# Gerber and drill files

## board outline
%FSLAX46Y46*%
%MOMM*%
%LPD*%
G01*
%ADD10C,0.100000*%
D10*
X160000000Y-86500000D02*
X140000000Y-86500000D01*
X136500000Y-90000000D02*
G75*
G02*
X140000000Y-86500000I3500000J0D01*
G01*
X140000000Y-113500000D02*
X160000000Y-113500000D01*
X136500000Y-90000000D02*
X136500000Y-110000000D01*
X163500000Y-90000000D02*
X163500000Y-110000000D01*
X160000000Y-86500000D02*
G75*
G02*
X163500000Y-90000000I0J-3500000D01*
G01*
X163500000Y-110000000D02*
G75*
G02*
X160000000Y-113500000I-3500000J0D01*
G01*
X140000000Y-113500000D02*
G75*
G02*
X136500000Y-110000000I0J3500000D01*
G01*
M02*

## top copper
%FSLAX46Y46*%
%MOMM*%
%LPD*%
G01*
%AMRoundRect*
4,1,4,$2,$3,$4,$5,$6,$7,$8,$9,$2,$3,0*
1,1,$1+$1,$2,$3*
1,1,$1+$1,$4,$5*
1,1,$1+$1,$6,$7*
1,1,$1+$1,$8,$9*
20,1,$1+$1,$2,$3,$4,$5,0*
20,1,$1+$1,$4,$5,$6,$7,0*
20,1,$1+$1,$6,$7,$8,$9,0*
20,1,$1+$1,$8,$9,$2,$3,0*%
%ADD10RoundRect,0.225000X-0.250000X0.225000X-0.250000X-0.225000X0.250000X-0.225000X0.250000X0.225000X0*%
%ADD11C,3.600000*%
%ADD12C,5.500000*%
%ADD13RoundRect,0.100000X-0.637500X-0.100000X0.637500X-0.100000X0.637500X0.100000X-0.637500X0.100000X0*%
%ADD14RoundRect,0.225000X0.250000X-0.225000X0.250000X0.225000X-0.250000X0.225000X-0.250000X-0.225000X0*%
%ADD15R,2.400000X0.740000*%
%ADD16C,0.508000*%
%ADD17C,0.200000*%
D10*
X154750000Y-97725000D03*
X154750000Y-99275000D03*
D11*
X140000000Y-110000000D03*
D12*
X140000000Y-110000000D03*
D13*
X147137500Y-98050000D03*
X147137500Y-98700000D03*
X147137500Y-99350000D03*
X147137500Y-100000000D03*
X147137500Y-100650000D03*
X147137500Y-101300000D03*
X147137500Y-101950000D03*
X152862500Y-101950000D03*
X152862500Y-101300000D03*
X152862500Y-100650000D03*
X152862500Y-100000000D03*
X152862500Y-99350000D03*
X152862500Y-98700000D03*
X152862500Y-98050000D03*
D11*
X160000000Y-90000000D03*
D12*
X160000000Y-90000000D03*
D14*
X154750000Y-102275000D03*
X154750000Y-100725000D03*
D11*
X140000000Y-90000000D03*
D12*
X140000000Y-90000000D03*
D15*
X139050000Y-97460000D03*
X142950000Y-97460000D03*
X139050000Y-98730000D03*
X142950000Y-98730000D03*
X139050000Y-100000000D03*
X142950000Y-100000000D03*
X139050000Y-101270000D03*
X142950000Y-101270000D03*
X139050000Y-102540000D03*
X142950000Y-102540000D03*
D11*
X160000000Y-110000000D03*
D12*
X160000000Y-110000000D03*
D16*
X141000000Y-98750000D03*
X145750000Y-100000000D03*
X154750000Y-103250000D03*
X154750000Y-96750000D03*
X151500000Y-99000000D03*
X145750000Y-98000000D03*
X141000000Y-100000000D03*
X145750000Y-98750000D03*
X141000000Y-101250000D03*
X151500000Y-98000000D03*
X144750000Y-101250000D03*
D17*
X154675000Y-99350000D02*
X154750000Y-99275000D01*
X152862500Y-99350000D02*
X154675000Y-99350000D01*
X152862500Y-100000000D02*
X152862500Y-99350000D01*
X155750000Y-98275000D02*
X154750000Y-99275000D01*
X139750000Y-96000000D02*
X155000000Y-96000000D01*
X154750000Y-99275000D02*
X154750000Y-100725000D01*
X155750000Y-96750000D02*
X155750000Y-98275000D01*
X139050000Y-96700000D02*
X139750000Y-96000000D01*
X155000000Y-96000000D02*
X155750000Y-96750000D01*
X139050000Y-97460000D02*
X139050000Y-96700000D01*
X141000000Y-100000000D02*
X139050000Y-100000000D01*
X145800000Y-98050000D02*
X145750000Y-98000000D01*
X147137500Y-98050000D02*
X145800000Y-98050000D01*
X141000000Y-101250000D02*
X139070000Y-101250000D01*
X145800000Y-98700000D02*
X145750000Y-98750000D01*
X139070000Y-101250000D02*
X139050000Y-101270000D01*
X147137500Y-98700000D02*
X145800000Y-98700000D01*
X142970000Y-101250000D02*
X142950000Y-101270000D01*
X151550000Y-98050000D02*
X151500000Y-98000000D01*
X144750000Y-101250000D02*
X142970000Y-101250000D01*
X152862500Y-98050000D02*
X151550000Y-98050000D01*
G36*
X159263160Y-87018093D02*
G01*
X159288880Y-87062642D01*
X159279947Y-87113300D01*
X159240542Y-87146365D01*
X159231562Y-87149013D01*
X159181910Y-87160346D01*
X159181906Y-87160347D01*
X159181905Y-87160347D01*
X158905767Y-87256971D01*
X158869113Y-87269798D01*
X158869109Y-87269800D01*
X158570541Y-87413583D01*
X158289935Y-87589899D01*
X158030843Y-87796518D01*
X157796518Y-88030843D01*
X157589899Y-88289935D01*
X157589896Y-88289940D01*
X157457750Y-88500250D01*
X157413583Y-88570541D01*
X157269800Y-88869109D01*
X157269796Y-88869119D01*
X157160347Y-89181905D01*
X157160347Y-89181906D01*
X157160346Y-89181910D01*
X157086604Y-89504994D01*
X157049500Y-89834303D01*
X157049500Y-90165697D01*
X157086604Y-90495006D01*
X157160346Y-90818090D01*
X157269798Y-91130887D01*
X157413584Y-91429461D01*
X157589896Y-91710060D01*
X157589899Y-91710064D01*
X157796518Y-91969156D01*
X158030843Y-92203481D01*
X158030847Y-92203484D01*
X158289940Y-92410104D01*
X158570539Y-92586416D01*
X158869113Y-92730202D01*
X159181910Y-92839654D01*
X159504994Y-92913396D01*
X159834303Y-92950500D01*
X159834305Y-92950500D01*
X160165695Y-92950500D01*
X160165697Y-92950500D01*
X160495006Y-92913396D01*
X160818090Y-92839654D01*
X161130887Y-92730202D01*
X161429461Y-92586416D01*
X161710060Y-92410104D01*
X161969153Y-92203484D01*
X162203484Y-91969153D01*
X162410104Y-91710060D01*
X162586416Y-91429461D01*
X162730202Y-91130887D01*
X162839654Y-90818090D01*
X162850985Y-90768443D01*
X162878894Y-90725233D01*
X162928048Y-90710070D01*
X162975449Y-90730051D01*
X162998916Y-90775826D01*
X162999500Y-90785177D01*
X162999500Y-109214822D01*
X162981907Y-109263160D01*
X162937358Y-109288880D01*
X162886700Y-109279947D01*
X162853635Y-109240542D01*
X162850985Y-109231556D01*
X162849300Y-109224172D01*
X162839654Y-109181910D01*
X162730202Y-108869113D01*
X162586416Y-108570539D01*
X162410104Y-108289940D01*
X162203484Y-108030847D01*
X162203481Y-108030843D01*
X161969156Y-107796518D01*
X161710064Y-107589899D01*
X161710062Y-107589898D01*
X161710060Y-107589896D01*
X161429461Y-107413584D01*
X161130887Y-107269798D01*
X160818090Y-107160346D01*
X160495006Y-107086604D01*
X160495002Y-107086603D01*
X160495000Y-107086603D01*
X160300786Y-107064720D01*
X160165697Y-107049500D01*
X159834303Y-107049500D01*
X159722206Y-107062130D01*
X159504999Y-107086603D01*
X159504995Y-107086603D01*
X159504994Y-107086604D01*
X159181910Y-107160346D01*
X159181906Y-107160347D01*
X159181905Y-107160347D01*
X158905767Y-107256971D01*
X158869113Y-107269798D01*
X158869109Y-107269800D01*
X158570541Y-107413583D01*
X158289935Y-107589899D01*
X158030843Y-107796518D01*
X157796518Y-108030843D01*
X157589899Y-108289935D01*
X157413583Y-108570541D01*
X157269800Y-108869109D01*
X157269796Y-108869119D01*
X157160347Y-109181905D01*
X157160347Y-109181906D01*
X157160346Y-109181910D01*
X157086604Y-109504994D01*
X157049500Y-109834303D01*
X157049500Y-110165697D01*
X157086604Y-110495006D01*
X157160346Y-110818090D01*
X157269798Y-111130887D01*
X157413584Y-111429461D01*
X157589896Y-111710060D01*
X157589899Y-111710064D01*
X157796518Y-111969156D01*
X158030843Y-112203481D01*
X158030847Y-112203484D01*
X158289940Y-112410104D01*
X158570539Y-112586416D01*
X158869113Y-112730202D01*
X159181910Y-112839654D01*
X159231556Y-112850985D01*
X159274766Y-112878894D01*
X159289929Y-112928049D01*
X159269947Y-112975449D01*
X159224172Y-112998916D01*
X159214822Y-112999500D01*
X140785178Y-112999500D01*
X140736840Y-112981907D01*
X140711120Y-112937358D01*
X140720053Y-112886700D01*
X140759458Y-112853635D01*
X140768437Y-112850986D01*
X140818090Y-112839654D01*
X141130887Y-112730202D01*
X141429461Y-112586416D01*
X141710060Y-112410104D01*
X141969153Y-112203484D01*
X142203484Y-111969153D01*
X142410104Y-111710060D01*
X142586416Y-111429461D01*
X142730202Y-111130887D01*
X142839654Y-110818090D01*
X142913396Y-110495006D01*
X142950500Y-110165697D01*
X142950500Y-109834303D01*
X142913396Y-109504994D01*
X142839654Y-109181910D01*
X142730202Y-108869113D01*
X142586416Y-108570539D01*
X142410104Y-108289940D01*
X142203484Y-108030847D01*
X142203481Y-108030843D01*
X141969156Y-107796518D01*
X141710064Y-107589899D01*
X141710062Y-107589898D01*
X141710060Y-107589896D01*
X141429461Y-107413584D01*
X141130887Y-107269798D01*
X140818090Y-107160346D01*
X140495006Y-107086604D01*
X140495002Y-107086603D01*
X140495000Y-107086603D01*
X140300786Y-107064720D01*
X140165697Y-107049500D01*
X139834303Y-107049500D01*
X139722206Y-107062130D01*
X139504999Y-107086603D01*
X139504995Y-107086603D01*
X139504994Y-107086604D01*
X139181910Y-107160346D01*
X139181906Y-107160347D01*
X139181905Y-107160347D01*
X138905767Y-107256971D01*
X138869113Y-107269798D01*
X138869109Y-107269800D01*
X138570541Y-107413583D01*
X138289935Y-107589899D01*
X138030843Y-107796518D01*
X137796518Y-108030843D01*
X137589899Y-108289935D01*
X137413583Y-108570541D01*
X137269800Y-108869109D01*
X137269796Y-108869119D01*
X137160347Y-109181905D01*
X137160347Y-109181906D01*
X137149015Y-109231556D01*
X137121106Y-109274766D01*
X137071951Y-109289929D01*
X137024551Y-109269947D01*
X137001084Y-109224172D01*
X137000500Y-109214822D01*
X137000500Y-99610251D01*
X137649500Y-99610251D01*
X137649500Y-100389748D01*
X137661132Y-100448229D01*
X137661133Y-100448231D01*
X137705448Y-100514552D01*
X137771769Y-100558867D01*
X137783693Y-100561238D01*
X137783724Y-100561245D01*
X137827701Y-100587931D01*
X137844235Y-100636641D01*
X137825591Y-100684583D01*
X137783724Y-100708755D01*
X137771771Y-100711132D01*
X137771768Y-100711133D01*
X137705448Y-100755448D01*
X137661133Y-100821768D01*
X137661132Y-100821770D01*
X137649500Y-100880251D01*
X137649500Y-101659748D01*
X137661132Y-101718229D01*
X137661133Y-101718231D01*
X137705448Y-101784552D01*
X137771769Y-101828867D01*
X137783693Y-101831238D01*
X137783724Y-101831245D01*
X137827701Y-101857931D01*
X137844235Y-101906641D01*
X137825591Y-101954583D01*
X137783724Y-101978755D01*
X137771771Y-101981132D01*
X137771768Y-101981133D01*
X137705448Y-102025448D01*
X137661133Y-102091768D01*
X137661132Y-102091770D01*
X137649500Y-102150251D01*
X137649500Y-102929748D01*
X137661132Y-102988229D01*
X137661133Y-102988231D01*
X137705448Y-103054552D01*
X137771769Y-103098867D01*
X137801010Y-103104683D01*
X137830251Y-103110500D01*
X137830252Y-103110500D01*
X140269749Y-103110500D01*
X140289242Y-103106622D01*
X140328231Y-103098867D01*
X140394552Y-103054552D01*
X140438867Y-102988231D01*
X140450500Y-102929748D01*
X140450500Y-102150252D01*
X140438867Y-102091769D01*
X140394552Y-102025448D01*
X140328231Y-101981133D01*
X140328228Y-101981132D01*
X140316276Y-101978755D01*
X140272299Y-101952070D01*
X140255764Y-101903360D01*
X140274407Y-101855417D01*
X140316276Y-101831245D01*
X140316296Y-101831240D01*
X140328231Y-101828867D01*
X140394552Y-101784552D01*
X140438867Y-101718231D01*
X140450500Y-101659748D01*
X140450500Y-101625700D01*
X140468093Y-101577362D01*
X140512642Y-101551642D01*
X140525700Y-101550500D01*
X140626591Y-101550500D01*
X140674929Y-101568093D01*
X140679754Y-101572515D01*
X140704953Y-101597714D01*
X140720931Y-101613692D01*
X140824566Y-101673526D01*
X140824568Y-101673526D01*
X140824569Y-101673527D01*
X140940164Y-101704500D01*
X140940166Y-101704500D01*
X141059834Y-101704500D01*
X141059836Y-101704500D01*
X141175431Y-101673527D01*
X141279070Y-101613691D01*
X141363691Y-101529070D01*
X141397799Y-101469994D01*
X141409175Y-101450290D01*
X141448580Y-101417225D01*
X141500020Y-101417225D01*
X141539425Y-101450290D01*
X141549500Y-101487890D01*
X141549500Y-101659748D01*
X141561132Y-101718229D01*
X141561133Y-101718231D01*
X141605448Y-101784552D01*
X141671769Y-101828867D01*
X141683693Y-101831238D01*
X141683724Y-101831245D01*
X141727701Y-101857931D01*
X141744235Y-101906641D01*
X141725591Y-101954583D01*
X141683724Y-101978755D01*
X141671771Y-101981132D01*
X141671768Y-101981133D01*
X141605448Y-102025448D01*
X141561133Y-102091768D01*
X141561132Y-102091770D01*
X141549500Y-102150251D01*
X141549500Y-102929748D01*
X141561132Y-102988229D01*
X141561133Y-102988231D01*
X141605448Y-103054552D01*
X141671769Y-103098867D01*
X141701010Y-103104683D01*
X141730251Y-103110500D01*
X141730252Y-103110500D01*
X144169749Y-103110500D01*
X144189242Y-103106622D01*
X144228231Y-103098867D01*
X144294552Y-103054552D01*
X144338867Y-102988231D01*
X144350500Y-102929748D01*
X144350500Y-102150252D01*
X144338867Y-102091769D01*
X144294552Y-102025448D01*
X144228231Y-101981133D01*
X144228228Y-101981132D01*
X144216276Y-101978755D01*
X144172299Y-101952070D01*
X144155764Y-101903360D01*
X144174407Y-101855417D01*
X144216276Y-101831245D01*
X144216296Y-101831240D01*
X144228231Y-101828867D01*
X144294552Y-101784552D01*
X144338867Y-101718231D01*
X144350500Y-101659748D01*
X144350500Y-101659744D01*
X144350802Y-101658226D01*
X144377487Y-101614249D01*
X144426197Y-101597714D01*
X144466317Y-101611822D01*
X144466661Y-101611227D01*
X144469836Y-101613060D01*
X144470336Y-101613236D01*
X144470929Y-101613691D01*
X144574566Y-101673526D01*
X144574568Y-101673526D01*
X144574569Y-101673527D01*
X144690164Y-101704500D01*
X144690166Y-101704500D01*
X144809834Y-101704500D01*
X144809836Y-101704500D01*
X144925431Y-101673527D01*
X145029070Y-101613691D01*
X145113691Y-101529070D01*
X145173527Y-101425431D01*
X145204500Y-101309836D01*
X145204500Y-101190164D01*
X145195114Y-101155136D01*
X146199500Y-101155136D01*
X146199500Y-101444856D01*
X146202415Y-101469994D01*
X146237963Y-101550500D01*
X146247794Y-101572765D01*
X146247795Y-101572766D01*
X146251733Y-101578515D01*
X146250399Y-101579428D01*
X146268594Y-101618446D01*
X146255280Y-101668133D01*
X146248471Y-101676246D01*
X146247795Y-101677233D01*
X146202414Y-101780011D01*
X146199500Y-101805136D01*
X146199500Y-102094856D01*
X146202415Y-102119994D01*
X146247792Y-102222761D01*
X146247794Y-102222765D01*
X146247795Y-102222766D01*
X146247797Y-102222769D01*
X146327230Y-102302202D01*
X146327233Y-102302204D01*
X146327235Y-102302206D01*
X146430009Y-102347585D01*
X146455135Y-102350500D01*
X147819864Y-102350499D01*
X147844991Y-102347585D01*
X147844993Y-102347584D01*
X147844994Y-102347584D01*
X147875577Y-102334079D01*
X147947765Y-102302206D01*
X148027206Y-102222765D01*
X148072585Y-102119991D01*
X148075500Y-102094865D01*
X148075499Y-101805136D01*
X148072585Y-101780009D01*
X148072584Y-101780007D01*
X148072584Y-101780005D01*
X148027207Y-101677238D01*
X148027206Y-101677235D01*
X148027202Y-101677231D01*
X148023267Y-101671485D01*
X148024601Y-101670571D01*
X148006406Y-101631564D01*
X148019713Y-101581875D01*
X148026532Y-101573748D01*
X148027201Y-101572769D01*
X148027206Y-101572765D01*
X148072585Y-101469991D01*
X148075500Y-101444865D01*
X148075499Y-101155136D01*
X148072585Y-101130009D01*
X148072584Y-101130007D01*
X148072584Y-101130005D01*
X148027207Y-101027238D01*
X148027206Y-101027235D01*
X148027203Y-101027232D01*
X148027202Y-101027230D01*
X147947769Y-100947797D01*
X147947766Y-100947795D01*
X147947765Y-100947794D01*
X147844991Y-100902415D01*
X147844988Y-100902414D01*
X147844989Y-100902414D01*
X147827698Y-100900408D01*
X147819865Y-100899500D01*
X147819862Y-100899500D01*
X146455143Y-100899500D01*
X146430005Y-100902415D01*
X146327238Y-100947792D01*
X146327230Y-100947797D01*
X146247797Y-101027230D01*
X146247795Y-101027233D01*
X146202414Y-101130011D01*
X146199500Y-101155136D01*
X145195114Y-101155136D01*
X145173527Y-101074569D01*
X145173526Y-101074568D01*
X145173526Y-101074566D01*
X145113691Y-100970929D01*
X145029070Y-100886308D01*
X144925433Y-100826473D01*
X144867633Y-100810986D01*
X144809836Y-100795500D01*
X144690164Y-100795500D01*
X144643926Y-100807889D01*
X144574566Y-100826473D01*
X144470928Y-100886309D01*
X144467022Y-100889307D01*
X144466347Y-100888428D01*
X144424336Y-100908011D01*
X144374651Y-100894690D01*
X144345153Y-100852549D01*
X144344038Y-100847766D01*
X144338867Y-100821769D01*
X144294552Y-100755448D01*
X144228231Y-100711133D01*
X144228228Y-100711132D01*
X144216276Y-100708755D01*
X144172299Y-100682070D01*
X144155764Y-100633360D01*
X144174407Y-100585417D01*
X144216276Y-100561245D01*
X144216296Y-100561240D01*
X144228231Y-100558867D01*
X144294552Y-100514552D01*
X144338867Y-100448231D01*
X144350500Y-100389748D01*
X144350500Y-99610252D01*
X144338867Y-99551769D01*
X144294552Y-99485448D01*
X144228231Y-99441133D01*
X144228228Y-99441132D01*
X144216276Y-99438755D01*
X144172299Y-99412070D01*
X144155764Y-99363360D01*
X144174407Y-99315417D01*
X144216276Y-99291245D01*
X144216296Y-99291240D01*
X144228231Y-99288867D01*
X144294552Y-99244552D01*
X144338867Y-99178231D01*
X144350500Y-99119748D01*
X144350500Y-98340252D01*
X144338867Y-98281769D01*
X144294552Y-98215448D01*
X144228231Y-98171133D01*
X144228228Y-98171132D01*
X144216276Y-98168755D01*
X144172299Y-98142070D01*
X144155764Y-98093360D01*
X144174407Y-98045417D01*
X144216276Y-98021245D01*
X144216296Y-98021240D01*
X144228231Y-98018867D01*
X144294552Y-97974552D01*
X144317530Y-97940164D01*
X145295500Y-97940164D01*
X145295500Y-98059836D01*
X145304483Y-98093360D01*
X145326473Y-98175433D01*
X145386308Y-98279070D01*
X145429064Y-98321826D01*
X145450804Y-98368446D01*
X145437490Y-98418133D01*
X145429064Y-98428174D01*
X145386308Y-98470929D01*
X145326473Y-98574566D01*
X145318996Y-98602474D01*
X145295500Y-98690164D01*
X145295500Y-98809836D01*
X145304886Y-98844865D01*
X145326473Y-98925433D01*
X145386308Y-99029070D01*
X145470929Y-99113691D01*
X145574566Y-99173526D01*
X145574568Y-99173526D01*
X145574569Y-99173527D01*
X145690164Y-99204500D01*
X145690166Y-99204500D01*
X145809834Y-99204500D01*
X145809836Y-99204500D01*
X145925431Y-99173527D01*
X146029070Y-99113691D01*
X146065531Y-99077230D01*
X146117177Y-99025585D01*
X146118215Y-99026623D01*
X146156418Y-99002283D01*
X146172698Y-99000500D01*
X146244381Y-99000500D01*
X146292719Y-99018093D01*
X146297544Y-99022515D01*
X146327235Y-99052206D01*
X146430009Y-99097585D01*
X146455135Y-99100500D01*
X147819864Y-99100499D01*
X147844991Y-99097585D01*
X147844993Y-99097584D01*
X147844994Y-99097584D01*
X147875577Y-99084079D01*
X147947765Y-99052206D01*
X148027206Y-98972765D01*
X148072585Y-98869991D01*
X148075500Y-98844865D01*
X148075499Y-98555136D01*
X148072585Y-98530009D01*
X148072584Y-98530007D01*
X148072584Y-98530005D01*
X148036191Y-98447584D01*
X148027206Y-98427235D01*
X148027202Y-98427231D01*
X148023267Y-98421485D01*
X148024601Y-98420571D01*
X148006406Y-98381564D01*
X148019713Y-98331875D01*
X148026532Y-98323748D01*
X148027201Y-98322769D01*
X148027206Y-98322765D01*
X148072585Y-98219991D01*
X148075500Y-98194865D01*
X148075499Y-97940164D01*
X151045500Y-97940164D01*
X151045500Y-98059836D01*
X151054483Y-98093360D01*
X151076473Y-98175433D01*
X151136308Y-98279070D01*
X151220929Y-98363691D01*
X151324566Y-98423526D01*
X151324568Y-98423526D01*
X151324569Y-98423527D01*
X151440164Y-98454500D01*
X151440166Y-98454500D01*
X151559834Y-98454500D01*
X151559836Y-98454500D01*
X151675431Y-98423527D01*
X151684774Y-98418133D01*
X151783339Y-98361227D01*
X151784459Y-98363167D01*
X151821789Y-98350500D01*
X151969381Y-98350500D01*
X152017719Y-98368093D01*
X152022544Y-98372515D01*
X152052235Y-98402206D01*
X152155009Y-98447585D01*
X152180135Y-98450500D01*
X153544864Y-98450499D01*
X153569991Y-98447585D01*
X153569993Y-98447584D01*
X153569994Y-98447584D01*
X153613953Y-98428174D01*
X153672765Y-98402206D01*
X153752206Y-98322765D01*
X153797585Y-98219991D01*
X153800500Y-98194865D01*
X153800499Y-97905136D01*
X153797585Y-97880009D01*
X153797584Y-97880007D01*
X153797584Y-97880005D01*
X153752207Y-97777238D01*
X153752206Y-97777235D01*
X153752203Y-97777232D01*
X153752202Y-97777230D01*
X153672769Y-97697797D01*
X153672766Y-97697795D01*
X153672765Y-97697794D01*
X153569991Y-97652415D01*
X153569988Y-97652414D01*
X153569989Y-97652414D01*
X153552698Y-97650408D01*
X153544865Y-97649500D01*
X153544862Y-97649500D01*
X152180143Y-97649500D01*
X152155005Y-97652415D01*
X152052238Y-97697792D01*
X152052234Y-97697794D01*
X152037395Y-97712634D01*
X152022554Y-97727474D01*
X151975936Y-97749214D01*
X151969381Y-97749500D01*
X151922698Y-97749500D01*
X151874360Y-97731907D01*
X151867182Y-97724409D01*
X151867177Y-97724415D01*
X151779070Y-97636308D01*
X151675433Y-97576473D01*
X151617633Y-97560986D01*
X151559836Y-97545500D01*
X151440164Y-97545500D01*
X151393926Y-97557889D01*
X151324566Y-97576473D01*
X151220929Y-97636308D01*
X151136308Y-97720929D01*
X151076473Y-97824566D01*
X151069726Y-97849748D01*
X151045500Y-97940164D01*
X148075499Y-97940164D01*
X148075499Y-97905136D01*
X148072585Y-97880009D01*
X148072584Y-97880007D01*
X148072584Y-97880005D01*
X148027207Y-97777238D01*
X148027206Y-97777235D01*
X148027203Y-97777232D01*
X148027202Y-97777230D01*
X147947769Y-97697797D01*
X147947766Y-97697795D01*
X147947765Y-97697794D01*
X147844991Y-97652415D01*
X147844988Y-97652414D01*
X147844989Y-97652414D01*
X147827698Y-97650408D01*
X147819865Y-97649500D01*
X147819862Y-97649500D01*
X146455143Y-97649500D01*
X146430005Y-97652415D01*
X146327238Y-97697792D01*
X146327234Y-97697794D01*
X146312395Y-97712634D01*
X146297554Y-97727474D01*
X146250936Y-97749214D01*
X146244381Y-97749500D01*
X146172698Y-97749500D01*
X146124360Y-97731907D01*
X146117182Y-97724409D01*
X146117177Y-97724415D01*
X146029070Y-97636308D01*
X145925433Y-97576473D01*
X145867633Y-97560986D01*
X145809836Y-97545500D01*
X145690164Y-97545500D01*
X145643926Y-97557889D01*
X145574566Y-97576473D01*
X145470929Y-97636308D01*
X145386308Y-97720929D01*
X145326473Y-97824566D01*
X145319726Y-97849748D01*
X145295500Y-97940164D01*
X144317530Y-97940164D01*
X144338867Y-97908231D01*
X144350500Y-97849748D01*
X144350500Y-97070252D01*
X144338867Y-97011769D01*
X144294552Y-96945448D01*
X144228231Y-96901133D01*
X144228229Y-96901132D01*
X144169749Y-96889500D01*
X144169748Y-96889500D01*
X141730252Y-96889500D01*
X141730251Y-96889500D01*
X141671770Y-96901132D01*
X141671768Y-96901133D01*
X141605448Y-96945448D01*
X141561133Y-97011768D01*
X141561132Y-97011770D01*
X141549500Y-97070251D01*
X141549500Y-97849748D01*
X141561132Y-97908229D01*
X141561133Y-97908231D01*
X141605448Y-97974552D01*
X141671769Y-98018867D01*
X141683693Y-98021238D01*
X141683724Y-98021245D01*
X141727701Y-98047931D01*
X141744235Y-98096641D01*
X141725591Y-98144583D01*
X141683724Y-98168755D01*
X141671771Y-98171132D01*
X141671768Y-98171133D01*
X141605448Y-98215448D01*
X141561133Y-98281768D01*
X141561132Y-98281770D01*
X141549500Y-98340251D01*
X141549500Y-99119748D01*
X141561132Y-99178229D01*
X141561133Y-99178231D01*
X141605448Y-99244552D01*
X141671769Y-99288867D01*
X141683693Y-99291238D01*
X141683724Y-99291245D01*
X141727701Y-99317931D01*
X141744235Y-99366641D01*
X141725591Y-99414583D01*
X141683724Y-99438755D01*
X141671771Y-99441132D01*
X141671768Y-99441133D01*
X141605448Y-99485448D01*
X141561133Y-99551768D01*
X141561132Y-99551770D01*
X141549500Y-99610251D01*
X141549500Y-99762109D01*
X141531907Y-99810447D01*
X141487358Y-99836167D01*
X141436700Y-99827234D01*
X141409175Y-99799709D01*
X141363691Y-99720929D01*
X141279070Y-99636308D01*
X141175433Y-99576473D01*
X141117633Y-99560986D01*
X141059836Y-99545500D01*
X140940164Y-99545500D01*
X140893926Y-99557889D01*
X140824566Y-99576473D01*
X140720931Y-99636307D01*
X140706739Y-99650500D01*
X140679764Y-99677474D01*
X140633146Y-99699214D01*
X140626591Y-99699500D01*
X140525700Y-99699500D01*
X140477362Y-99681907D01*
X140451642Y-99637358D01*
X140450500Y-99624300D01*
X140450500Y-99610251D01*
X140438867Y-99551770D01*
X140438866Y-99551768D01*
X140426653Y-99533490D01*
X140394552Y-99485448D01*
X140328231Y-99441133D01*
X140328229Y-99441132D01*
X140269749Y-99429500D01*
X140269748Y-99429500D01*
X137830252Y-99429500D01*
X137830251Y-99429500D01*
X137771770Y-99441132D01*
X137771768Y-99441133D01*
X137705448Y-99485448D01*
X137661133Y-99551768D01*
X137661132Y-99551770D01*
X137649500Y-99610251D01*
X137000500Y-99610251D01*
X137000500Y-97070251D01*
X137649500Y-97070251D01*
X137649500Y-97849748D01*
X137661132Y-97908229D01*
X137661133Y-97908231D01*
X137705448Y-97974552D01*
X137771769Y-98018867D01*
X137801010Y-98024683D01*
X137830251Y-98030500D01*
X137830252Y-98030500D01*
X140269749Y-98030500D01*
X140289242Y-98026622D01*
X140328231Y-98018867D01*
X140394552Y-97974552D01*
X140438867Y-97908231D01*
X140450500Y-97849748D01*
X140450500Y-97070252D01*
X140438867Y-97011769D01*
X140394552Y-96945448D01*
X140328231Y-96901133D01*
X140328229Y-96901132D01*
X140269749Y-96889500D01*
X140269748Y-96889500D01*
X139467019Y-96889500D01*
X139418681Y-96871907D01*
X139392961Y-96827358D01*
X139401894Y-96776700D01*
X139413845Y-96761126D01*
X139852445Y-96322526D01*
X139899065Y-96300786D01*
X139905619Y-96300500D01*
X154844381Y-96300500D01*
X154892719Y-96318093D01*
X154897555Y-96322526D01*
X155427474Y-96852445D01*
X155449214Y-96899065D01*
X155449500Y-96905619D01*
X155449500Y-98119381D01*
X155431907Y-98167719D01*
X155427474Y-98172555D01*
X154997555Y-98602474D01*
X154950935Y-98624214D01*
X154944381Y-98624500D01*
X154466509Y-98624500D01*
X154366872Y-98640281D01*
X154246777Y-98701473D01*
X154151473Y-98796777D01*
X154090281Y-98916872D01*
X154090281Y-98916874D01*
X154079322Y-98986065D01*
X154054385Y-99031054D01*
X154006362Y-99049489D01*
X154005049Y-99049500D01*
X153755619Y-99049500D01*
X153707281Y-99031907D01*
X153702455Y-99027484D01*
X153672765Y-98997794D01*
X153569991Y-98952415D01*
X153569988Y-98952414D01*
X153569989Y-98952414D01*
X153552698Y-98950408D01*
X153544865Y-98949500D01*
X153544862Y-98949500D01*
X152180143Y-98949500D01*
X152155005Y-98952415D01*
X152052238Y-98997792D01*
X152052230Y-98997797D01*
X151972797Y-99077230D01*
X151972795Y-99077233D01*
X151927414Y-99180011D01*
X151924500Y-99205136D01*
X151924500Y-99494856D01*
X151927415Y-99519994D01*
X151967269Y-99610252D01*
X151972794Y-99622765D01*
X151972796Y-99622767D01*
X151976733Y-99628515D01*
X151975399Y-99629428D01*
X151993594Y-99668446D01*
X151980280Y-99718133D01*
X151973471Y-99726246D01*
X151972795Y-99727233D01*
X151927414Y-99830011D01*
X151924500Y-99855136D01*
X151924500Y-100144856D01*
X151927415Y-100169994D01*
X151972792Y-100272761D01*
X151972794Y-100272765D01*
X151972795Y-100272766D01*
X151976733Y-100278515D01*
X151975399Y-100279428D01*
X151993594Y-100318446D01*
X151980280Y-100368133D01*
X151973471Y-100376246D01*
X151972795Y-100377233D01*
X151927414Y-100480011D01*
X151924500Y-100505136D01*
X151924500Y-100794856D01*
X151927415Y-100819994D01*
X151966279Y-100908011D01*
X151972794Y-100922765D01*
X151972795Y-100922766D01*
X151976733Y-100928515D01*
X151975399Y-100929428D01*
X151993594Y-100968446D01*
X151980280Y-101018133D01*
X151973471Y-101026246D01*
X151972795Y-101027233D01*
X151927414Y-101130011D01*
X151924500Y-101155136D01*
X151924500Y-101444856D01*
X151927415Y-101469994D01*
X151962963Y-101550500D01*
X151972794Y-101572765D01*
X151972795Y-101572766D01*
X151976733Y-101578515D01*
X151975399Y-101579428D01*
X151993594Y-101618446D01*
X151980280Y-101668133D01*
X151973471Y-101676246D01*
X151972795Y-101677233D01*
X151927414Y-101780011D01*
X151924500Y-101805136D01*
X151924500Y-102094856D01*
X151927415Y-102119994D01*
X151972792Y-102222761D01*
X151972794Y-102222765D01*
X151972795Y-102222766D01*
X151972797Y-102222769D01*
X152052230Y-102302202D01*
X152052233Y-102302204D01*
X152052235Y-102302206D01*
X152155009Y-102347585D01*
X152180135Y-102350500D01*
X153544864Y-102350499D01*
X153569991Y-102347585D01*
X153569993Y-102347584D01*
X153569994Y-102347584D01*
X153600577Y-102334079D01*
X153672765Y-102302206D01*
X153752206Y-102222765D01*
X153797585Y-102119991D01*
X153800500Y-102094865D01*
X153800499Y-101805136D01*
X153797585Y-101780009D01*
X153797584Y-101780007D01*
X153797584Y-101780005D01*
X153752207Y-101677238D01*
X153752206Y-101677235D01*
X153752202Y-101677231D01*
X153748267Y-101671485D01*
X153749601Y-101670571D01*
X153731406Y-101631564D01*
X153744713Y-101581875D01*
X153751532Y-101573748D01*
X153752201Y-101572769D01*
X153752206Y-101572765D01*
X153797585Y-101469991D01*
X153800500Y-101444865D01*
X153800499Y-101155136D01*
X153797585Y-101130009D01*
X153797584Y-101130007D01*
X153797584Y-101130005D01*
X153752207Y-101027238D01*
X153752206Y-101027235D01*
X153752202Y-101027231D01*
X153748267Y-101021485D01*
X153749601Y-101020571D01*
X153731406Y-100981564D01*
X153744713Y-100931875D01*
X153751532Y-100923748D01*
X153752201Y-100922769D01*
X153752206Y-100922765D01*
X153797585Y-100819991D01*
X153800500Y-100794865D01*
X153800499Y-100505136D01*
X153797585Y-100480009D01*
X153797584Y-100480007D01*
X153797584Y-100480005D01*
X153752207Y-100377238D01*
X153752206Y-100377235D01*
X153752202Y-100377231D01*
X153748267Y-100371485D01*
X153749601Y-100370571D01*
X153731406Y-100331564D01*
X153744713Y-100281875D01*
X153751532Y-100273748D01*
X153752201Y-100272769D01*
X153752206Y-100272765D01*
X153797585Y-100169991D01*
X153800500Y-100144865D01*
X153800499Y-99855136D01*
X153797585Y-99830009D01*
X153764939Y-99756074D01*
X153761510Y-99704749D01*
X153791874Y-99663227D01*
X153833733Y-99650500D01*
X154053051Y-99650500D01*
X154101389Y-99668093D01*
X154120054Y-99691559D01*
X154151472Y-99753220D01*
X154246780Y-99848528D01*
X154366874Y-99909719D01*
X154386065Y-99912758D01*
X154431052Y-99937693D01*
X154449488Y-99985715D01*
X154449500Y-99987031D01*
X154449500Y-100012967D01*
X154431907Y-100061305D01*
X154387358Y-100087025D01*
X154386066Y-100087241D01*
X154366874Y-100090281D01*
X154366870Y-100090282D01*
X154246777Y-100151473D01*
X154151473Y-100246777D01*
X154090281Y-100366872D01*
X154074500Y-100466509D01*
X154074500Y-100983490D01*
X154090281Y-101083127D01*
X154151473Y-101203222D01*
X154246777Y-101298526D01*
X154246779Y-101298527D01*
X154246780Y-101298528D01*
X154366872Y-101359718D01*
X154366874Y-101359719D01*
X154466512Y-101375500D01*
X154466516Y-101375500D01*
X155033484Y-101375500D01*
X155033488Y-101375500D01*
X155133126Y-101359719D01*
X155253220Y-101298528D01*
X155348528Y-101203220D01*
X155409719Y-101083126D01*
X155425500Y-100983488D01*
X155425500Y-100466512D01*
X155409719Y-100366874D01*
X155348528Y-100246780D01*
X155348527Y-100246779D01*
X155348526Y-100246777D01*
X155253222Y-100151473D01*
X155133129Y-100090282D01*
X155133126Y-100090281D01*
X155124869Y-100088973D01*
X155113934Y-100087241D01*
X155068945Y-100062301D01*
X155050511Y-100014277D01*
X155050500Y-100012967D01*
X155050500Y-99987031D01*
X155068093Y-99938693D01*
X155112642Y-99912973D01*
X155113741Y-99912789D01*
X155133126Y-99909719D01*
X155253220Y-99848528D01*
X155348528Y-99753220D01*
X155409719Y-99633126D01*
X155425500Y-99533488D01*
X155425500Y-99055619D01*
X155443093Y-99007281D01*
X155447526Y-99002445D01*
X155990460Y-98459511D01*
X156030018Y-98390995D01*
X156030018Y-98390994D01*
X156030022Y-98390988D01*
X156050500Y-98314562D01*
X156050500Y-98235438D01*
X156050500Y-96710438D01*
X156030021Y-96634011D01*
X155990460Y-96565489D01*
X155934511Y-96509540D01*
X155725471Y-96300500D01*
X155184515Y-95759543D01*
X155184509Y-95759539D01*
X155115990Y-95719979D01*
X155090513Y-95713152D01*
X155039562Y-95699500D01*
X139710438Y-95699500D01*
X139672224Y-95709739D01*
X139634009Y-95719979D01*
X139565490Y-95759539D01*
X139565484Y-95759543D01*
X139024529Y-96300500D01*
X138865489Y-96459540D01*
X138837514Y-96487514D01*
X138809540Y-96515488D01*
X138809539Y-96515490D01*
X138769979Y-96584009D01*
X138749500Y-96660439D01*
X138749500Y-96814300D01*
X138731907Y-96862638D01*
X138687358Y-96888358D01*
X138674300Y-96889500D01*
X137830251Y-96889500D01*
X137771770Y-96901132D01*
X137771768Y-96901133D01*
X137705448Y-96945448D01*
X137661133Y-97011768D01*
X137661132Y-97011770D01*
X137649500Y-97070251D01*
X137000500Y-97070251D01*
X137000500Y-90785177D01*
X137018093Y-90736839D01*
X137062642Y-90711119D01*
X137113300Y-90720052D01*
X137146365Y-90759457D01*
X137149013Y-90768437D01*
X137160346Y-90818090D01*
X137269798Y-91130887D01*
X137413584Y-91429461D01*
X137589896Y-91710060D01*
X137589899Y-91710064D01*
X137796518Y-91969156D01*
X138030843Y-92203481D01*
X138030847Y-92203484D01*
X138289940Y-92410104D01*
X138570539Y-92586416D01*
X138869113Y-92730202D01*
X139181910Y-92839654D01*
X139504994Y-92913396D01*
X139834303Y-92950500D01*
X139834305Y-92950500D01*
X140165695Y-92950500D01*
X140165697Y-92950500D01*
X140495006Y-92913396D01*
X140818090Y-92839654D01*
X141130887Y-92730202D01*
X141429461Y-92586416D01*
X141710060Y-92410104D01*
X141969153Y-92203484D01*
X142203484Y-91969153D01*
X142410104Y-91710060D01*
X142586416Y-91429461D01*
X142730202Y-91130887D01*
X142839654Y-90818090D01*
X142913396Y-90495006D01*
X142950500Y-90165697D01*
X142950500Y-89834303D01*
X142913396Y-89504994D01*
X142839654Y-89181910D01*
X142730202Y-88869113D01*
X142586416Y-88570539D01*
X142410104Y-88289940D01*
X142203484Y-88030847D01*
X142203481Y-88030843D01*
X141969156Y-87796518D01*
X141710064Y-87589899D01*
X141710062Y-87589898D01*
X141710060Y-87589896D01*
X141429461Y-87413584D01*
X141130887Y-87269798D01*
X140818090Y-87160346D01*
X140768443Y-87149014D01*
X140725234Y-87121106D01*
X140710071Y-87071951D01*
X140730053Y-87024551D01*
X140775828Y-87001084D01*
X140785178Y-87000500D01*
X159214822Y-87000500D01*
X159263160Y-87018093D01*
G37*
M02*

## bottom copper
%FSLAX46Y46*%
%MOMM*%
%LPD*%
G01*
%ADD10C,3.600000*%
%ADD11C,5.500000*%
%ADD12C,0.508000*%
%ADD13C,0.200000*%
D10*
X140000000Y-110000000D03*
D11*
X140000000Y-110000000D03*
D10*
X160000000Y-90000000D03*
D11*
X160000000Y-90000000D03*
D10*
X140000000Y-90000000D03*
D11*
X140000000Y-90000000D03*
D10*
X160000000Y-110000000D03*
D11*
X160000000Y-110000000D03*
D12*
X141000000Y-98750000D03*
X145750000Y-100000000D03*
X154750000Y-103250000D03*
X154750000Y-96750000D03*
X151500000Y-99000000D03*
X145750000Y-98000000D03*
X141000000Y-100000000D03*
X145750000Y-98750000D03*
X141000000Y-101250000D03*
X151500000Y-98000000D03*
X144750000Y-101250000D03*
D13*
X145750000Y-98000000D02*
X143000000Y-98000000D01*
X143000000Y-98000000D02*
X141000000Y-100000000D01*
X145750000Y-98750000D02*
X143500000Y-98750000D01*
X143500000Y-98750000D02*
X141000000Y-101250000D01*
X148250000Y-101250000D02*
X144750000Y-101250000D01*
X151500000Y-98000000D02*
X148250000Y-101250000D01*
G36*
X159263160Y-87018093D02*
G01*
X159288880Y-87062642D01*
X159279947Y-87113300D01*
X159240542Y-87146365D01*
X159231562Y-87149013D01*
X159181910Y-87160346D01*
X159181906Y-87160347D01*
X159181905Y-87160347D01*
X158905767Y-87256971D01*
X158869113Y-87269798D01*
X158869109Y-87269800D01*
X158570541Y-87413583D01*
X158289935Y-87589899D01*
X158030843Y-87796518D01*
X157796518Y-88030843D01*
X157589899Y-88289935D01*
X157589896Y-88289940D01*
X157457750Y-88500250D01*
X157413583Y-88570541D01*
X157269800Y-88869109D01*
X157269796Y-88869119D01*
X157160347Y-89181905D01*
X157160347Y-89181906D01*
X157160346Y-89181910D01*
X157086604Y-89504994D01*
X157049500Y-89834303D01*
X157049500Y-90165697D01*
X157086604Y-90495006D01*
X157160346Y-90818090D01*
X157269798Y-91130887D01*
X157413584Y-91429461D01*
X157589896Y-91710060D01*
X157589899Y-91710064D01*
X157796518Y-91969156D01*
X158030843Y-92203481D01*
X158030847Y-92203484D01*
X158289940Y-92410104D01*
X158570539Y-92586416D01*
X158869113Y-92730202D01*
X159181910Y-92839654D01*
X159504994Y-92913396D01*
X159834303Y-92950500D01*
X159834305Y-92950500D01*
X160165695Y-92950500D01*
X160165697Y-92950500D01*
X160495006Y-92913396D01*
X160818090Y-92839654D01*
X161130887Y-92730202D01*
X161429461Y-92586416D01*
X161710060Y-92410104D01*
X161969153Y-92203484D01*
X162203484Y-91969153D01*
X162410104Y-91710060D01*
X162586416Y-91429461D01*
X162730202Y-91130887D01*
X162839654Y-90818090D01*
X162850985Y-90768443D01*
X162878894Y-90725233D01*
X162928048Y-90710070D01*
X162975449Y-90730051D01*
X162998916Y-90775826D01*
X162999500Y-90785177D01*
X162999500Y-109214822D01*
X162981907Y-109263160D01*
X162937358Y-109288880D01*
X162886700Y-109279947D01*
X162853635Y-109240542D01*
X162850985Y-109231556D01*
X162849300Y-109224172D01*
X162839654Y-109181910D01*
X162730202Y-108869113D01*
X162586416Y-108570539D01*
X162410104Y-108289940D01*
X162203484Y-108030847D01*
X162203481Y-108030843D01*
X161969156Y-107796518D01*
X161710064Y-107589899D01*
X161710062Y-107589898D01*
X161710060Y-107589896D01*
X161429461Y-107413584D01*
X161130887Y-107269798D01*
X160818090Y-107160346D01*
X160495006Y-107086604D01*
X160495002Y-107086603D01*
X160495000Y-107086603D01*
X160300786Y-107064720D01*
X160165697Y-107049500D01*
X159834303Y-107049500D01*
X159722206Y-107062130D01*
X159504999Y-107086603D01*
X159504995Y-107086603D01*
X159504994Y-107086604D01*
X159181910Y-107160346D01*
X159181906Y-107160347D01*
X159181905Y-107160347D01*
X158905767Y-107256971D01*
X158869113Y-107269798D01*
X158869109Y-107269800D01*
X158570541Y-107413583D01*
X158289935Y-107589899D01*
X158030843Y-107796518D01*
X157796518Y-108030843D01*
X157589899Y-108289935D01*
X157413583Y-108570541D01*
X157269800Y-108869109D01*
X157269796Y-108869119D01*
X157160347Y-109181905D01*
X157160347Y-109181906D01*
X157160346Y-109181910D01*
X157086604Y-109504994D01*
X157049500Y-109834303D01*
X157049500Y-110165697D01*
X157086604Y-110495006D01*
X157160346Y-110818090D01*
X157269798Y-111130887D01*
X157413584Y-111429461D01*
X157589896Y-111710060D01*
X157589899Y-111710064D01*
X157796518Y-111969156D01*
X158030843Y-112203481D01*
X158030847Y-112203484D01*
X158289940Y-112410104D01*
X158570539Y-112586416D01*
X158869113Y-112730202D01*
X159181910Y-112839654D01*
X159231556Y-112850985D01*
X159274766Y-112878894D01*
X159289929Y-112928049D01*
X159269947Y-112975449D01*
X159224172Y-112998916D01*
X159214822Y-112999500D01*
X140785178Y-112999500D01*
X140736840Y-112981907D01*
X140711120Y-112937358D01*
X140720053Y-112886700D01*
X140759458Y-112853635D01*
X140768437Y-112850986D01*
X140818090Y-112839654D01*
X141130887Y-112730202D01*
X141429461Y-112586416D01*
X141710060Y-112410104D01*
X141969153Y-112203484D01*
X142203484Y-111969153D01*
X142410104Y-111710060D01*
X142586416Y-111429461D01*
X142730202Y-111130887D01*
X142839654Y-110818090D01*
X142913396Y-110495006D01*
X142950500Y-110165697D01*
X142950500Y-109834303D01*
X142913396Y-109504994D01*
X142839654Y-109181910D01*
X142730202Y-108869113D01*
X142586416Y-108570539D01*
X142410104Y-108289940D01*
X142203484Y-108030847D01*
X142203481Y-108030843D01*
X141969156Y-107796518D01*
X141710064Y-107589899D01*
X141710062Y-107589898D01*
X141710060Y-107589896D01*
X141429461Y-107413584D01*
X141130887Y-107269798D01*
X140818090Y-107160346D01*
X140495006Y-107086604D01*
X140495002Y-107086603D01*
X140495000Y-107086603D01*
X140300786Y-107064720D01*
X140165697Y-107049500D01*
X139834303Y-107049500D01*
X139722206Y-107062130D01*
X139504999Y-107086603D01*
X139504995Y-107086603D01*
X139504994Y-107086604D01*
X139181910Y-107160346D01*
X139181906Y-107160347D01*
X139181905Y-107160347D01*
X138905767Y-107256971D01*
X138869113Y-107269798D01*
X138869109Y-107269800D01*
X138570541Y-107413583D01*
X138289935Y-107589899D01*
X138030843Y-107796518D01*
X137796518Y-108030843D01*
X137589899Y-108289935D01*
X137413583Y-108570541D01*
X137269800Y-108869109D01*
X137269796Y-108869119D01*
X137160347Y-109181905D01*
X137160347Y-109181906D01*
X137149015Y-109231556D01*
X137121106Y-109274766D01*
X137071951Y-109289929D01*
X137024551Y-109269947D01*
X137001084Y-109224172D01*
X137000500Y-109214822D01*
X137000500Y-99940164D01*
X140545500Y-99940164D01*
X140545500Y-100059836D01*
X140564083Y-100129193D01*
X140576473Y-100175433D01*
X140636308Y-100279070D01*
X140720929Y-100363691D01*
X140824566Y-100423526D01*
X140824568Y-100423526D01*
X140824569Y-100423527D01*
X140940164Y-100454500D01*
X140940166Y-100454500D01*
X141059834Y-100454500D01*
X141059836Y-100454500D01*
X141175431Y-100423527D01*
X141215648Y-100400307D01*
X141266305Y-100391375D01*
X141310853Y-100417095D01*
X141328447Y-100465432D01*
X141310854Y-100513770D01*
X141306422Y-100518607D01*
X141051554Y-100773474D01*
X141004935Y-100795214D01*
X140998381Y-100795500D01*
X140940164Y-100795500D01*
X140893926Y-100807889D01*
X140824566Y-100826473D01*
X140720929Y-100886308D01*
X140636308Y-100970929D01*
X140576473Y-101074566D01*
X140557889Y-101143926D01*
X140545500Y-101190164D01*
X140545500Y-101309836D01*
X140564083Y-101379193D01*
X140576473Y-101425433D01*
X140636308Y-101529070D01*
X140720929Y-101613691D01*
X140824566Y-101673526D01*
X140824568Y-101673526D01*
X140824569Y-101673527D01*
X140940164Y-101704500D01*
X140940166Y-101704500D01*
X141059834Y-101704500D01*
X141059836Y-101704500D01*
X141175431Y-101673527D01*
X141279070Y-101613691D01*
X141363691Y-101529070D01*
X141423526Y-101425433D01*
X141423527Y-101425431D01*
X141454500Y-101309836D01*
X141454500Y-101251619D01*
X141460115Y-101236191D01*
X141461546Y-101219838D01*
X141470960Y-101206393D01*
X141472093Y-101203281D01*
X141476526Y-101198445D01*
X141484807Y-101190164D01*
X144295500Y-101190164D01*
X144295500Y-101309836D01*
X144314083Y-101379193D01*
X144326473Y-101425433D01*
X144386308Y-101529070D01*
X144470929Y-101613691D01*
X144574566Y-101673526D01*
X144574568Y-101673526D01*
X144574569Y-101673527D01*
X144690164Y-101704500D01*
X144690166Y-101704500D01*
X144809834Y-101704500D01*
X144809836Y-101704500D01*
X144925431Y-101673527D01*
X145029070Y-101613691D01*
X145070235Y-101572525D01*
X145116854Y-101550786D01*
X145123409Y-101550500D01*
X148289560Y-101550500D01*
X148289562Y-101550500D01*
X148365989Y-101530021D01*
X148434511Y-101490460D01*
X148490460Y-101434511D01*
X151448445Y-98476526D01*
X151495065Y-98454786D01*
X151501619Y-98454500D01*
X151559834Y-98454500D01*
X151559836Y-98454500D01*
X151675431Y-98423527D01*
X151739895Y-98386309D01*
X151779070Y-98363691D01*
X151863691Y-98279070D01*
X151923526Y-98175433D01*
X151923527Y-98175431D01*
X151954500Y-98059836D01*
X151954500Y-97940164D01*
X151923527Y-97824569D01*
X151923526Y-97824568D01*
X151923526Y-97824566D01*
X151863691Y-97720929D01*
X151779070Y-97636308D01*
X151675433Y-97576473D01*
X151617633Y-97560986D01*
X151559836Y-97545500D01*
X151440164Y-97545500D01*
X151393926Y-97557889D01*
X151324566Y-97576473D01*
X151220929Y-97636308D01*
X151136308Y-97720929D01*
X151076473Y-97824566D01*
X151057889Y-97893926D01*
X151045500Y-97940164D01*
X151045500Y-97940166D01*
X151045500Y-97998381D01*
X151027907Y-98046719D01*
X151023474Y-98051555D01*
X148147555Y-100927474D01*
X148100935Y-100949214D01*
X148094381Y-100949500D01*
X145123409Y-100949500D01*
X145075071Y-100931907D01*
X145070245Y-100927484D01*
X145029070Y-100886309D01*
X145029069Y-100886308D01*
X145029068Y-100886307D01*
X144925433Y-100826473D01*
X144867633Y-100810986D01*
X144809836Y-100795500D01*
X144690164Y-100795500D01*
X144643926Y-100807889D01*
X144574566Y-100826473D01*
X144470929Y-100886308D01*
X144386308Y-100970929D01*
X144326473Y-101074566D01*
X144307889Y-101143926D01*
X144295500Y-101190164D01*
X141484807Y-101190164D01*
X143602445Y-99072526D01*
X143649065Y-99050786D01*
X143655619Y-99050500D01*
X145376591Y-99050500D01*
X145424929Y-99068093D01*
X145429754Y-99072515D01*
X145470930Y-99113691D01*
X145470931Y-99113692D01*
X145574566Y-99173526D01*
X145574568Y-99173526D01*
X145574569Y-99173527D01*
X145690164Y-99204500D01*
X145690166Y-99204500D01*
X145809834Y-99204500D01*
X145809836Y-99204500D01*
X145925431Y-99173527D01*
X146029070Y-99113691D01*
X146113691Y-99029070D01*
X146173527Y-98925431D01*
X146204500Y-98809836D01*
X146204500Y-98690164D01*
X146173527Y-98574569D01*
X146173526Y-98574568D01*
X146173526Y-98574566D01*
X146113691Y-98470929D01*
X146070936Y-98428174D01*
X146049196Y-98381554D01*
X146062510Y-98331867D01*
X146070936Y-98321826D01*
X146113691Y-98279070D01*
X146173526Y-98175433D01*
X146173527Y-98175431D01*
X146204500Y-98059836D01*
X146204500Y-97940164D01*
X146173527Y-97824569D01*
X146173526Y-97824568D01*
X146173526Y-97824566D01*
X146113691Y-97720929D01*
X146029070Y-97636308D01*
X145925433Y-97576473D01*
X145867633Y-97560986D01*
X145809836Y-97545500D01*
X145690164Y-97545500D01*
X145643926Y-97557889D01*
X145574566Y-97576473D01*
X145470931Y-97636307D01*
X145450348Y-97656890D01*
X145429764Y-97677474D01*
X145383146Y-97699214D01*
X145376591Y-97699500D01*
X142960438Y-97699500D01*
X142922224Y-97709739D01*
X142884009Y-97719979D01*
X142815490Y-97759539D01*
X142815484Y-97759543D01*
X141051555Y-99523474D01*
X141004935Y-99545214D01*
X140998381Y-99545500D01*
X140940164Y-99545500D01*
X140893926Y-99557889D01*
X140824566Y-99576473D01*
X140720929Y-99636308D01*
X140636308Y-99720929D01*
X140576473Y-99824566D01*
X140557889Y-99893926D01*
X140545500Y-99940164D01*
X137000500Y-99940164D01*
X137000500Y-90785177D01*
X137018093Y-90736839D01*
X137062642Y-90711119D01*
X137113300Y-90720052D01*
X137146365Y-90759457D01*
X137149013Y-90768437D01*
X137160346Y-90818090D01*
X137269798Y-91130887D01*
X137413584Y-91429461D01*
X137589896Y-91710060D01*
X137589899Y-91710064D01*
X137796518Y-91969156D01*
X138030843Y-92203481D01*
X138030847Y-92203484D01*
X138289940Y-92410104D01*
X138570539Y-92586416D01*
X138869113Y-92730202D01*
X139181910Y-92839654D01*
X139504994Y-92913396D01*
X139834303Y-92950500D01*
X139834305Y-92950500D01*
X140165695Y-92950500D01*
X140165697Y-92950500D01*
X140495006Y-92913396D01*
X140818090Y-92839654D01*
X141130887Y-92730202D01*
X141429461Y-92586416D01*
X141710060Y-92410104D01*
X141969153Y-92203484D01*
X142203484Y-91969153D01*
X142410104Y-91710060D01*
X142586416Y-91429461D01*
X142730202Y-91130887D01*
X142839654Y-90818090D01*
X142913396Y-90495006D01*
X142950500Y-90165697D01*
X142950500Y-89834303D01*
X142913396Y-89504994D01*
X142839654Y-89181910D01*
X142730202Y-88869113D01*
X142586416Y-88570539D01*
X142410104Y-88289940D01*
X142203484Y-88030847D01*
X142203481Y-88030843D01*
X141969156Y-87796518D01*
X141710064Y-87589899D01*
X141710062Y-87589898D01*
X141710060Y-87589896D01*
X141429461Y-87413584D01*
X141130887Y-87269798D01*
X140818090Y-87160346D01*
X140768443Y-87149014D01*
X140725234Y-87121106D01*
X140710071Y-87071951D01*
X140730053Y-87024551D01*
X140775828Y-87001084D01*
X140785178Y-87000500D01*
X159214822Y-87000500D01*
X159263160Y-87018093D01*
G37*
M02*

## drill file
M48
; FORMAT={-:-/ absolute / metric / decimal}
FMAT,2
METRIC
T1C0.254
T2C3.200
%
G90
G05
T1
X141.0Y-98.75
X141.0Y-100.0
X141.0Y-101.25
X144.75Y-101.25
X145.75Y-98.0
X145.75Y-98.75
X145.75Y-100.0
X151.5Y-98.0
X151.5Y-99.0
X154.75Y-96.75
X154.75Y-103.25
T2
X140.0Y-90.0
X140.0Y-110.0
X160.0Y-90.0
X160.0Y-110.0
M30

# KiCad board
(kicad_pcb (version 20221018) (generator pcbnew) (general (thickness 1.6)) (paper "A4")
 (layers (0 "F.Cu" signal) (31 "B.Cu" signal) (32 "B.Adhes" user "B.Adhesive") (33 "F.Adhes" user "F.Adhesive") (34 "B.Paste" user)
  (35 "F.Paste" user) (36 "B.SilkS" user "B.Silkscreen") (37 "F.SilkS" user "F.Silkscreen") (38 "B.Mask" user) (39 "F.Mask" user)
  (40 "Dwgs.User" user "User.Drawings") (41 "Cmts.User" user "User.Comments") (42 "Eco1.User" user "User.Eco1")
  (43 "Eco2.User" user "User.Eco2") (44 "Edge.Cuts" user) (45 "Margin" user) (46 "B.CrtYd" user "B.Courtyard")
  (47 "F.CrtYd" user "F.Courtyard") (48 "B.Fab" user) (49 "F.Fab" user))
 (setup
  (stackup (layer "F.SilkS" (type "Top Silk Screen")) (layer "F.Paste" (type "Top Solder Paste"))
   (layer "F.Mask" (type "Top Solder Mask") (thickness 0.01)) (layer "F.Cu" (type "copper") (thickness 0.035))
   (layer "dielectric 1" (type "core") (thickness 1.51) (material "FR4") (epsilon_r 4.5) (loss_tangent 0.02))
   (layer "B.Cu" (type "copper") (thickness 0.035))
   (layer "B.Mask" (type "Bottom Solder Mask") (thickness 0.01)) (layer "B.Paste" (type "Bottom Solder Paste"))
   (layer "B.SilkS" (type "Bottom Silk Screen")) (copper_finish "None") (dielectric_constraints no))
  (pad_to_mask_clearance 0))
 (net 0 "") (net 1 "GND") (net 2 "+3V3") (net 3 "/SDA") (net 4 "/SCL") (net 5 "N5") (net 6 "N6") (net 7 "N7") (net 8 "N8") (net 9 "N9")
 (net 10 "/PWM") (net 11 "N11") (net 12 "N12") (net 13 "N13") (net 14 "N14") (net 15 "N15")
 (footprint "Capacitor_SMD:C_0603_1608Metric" (layer "F.Cu") (at 154.75 98.5 -90)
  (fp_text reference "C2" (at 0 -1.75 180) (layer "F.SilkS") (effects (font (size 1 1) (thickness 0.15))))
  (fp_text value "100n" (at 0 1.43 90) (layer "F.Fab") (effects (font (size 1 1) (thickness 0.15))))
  (pad "1" smd roundrect (at -0.775 0 270) (size 0.9 0.95) (layers "F.Cu" "F.Paste" "F.Mask") (roundrect_rratio 0.25) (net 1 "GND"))
  (pad "2" smd roundrect (at 0.775 0 270) (size 0.9 0.95) (layers "F.Cu" "F.Paste" "F.Mask") (roundrect_rratio 0.25) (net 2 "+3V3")))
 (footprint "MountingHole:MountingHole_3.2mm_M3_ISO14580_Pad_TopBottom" (layer "F.Cu") (at 140 110)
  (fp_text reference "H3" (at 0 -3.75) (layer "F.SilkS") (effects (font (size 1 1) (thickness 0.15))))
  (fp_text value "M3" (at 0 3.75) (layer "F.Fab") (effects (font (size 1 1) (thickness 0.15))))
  (pad "1" thru_hole circle (at 0 0) (size 3.6 3.6) (drill 3.2) (layers "*.Cu" "*.Mask"))
  (pad "1" connect circle (at 0 0) (size 5.5 5.5) (layers "F.Cu" "F.Mask"))
  (pad "1" connect circle (at 0 0) (size 5.5 5.5) (layers "B.Cu" "B.Mask")))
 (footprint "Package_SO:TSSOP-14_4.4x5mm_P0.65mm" (layer "F.Cu") (at 150 100)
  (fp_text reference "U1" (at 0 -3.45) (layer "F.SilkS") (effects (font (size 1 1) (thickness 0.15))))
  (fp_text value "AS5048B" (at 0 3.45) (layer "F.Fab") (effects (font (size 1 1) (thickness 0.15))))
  (pad "1" smd roundrect (at -2.8625 -1.95) (size 1.475 0.4) (layers "F.Cu" "F.Paste" "F.Mask") (roundrect_rratio 0.25) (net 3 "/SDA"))
  (pad "2" smd roundrect (at -2.8625 -1.3) (size 1.475 0.4) (layers "F.Cu" "F.Paste" "F.Mask") (roundrect_rratio 0.25) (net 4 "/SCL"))
  (pad "3" smd roundrect (at -2.8625 -0.65) (size 1.475 0.4) (layers "F.Cu" "F.Paste" "F.Mask") (roundrect_rratio 0.25) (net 1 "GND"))
  (pad "4" smd roundrect (at -2.8625 0) (size 1.475 0.4) (layers "F.Cu" "F.Paste" "F.Mask") (roundrect_rratio 0.25) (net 1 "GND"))
  (pad "5" smd roundrect (at -2.8625 0.65) (size 1.475 0.4) (layers "F.Cu" "F.Paste" "F.Mask") (roundrect_rratio 0.25) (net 1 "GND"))
  (pad "6" smd roundrect (at -2.8625 1.3) (size 1.475 0.4) (layers "F.Cu" "F.Paste" "F.Mask") (roundrect_rratio 0.25) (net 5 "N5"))
  (pad "7" smd roundrect (at -2.8625 1.95) (size 1.475 0.4) (layers "F.Cu" "F.Paste" "F.Mask") (roundrect_rratio 0.25) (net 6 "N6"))
  (pad "8" smd roundrect (at 2.8625 1.95) (size 1.475 0.4) (layers "F.Cu" "F.Paste" "F.Mask") (roundrect_rratio 0.25) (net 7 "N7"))
  (pad "9" smd roundrect (at 2.8625 1.3) (size 1.475 0.4) (layers "F.Cu" "F.Paste" "F.Mask") (roundrect_rratio 0.25) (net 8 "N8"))
  (pad "10" smd roundrect (at 2.8625 0.65) (size 1.475 0.4) (layers "F.Cu" "F.Paste" "F.Mask") (roundrect_rratio 0.25) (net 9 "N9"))
  (pad "11" smd roundrect (at 2.8625 0) (size 1.475 0.4) (layers "F.Cu" "F.Paste" "F.Mask") (roundrect_rratio 0.25) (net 2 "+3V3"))
  (pad "12" smd roundrect (at 2.8625 -0.65) (size 1.475 0.4) (layers "F.Cu" "F.Paste" "F.Mask") (roundrect_rratio 0.25) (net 2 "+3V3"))
  (pad "13" smd roundrect (at 2.8625 -1.3) (size 1.475 0.4) (layers "F.Cu" "F.Paste" "F.Mask") (roundrect_rratio 0.25) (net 1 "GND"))
  (pad "14" smd roundrect (at 2.8625 -1.95) (size 1.475 0.4) (layers "F.Cu" "F.Paste" "F.Mask") (roundrect_rratio 0.25) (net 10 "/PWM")))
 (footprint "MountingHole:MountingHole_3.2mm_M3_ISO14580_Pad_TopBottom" (layer "F.Cu") (at 160 90)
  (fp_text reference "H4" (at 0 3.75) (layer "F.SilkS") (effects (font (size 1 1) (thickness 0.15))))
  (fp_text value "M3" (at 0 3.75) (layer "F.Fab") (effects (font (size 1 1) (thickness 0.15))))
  (pad "1" thru_hole circle (at 0 0) (size 3.6 3.6) (drill 3.2) (layers "*.Cu" "*.Mask"))
  (pad "1" connect circle (at 0 0) (size 5.5 5.5) (layers "F.Cu" "F.Mask"))
  (pad "1" connect circle (at 0 0) (size 5.5 5.5) (layers "B.Cu" "B.Mask")))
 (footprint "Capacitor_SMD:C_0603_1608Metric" (layer "F.Cu") (at 154.75 101.5 90)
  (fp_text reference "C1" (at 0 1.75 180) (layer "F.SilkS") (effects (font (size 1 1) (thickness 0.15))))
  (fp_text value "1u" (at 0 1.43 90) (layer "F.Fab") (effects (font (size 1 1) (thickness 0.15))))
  (pad "1" smd roundrect (at -0.775 0 90) (size 0.9 0.95) (layers "F.Cu" "F.Paste" "F.Mask") (roundrect_rratio 0.25) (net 1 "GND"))
  (pad "2" smd roundrect (at 0.775 0 90) (size 0.9 0.95) (layers "F.Cu" "F.Paste" "F.Mask") (roundrect_rratio 0.25) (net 2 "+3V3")))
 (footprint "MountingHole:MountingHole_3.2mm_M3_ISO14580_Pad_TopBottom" (layer "F.Cu") (at 140 90)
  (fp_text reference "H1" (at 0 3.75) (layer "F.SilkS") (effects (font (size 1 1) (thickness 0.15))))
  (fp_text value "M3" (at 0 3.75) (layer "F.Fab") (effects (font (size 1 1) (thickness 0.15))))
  (pad "1" thru_hole circle (at 0 0) (size 3.6 3.6) (drill 3.2) (layers "*.Cu" "*.Mask"))
  (pad "1" connect circle (at 0 0) (size 5.5 5.5) (layers "F.Cu" "F.Mask"))
  (pad "1" connect circle (at 0 0) (size 5.5 5.5) (layers "B.Cu" "B.Mask")))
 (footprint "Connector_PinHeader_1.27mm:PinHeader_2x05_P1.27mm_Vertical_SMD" (layer "F.Cu") (at 141 100)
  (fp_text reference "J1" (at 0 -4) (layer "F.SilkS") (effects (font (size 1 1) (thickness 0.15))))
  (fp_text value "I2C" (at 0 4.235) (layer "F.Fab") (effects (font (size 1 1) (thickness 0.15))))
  (pad "1" smd rect (at -1.95 -2.54) (size 2.4 0.74) (layers "F.Cu" "F.Paste" "F.Mask") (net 2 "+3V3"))
  (pad "2" smd rect (at 1.95 -2.54) (size 2.4 0.74) (layers "F.Cu" "F.Paste" "F.Mask") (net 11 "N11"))
  (pad "3" smd rect (at -1.95 -1.27) (size 2.4 0.74) (layers "F.Cu" "F.Paste" "F.Mask") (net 1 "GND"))
  (pad "4" smd rect (at 1.95 -1.27) (size 2.4 0.74) (layers "F.Cu" "F.Paste" "F.Mask") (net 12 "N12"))
  (pad "5" smd rect (at -1.95 0) (size 2.4 0.74) (layers "F.Cu" "F.Paste" "F.Mask") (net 3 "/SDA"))
  (pad "6" smd rect (at 1.95 0) (size 2.4 0.74) (layers "F.Cu" "F.Paste" "F.Mask") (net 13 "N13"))
  (pad "7" smd rect (at -1.95 1.27) (size 2.4 0.74) (layers "F.Cu" "F.Paste" "F.Mask") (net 4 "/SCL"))
  (pad "8" smd rect (at 1.95 1.27) (size 2.4 0.74) (layers "F.Cu" "F.Paste" "F.Mask") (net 10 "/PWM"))
  (pad "9" smd rect (at -1.95 2.54) (size 2.4 0.74) (layers "F.Cu" "F.Paste" "F.Mask") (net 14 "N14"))
  (pad "10" smd rect (at 1.95 2.54) (size 2.4 0.74) (layers "F.Cu" "F.Paste" "F.Mask") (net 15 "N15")))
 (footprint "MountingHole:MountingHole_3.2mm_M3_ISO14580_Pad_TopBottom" (layer "F.Cu") (at 160 110)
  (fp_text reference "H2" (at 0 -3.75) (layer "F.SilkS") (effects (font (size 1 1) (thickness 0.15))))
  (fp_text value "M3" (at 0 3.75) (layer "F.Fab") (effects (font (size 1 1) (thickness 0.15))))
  (pad "1" thru_hole circle (at 0 0) (size 3.6 3.6) (drill 3.2) (layers "*.Cu" "*.Mask"))
  (pad "1" connect circle (at 0 0) (size 5.5 5.5) (layers "F.Cu" "F.Mask"))
  (pad "1" connect circle (at 0 0) (size 5.5 5.5) (layers "B.Cu" "B.Mask")))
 (gr_line (start 160 86.5) (end 140 86.5) (stroke (width 0.1) (type solid)) (layer "Edge.Cuts"))
 (gr_arc (start 136.5 90) (mid 137.525126 87.525126) (end 140 86.5) (stroke (width 0.1) (type solid)) (layer "Edge.Cuts"))
 (gr_line (start 140 113.5) (end 160 113.5) (stroke (width 0.1) (type solid)) (layer "Edge.Cuts"))
 (gr_line (start 136.5 90) (end 136.5 110) (stroke (width 0.1) (type solid)) (layer "Edge.Cuts"))
 (gr_line (start 163.5 90) (end 163.5 110) (stroke (width 0.1) (type solid)) (layer "Edge.Cuts"))
 (gr_arc (start 160 86.5) (mid 162.474874 87.525126) (end 163.5 90) (stroke (width 0.1) (type solid)) (layer "Edge.Cuts"))
 (gr_arc (start 163.5 110) (mid 162.474874 112.474874) (end 160 113.5) (stroke (width 0.1) (type solid)) (layer "Edge.Cuts"))
 (gr_arc (start 140 113.5) (mid 137.525126 112.474874) (end 136.5 110) (stroke (width 0.1) (type solid)) (layer "Edge.Cuts"))
 (via (at 141 98.75) (size 0.508) (drill 0.254) (layers "F.Cu" "B.Cu") (free) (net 1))
 (via (at 145.75 100) (size 0.508) (drill 0.254) (layers "F.Cu" "B.Cu") (free) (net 1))
 (via (at 154.75 103.25) (size 0.508) (drill 0.254) (layers "F.Cu" "B.Cu") (free) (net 1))
 (via (at 154.75 96.75) (size 0.508) (drill 0.254) (layers "F.Cu" "B.Cu") (free) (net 1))
 (via (at 151.5 99) (size 0.508) (drill 0.254) (layers "F.Cu" "B.Cu") (free) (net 1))
 (segment (start 154.675 99.35) (end 154.75 99.275) (width 0.2) (layer "F.Cu") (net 2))
 (segment (start 152.8625 99.35) (end 154.675 99.35) (width 0.2) (layer "F.Cu") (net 2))
 (segment (start 152.8625 100) (end 152.8625 99.35) (width 0.2) (layer "F.Cu") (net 2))
 (segment (start 155.75 98.275) (end 154.75 99.275) (width 0.2) (layer "F.Cu") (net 2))
 (segment (start 139.75 96) (end 155 96) (width 0.2) (layer "F.Cu") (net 2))
 (segment (start 154.75 99.275) (end 154.75 100.725) (width 0.2) (layer "F.Cu") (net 2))
 (segment (start 155.75 96.75) (end 155.75 98.275) (width 0.2) (layer "F.Cu") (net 2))
 (segment (start 139.05 96.7) (end 139.75 96) (width 0.2) (layer "F.Cu") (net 2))
 (segment (start 155 96) (end 155.75 96.75) (width 0.2) (layer "F.Cu") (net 2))
 (segment (start 139.05 97.46) (end 139.05 96.7) (width 0.2) (layer "F.Cu") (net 2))
 (segment (start 141 100) (end 139.05 100) (width 0.2) (layer "F.Cu") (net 3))
 (segment (start 145.8 98.05) (end 145.75 98) (width 0.2) (layer "F.Cu") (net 3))
 (segment (start 147.1375 98.05) (end 145.8 98.05) (width 0.2) (layer "F.Cu") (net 3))
 (via (at 145.75 98) (size 0.508) (drill 0.254) (layers "F.Cu" "B.Cu") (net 3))
 (via (at 141 100) (size 0.508) (drill 0.254) (layers "F.Cu" "B.Cu") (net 3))
 (segment (start 145.75 98) (end 143 98) (width 0.2) (layer "B.Cu") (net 3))
 (segment (start 143 98) (end 141 100) (width 0.2) (layer "B.Cu") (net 3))
 (segment (start 141 101.25) (end 139.07 101.25) (width 0.2) (layer "F.Cu") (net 4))
 (segment (start 145.8 98.7) (end 145.75 98.75) (width 0.2) (layer "F.Cu") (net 4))
 (segment (start 139.07 101.25) (end 139.05 101.27) (width 0.2) (layer "F.Cu") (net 4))
 (segment (start 147.1375 98.7) (end 145.8 98.7) (width 0.2) (layer "F.Cu") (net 4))
 (via (at 145.75 98.75) (size 0.508) (drill 0.254) (layers "F.Cu" "B.Cu") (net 4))
 (via (at 141 101.25) (size 0.508) (drill 0.254) (layers "F.Cu" "B.Cu") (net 4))
 (segment (start 145.75 98.75) (end 143.5 98.75) (width 0.2) (layer "B.Cu") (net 4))
 (segment (start 143.5 98.75) (end 141 101.25) (width 0.2) (layer "B.Cu") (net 4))
 (segment (start 142.97 101.25) (end 142.95 101.27) (width 0.2) (layer "F.Cu") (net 10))
 (segment (start 151.55 98.05) (end 151.5 98) (width 0.2) (layer "F.Cu") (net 10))
 (segment (start 144.75 101.25) (end 142.97 101.25) (width 0.2) (layer "F.Cu") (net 10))
 (segment (start 152.8625 98.05) (end 151.55 98.05) (width 0.2) (layer "F.Cu") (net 10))
 (via (at 151.5 98) (size 0.508) (drill 0.254) (layers "F.Cu" "B.Cu") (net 10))
 (via (at 144.75 101.25) (size 0.508) (drill 0.254) (layers "F.Cu" "B.Cu") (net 10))
 (segment (start 148.25 101.25) (end 144.75 101.25) (width 0.2) (layer "B.Cu") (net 10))
 (segment (start 151.5 98) (end 148.25 101.25) (width 0.2) (layer "B.Cu") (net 10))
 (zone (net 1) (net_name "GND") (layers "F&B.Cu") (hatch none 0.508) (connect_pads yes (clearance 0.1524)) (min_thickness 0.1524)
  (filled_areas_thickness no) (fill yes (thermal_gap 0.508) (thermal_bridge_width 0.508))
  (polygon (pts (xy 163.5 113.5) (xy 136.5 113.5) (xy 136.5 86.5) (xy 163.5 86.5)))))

